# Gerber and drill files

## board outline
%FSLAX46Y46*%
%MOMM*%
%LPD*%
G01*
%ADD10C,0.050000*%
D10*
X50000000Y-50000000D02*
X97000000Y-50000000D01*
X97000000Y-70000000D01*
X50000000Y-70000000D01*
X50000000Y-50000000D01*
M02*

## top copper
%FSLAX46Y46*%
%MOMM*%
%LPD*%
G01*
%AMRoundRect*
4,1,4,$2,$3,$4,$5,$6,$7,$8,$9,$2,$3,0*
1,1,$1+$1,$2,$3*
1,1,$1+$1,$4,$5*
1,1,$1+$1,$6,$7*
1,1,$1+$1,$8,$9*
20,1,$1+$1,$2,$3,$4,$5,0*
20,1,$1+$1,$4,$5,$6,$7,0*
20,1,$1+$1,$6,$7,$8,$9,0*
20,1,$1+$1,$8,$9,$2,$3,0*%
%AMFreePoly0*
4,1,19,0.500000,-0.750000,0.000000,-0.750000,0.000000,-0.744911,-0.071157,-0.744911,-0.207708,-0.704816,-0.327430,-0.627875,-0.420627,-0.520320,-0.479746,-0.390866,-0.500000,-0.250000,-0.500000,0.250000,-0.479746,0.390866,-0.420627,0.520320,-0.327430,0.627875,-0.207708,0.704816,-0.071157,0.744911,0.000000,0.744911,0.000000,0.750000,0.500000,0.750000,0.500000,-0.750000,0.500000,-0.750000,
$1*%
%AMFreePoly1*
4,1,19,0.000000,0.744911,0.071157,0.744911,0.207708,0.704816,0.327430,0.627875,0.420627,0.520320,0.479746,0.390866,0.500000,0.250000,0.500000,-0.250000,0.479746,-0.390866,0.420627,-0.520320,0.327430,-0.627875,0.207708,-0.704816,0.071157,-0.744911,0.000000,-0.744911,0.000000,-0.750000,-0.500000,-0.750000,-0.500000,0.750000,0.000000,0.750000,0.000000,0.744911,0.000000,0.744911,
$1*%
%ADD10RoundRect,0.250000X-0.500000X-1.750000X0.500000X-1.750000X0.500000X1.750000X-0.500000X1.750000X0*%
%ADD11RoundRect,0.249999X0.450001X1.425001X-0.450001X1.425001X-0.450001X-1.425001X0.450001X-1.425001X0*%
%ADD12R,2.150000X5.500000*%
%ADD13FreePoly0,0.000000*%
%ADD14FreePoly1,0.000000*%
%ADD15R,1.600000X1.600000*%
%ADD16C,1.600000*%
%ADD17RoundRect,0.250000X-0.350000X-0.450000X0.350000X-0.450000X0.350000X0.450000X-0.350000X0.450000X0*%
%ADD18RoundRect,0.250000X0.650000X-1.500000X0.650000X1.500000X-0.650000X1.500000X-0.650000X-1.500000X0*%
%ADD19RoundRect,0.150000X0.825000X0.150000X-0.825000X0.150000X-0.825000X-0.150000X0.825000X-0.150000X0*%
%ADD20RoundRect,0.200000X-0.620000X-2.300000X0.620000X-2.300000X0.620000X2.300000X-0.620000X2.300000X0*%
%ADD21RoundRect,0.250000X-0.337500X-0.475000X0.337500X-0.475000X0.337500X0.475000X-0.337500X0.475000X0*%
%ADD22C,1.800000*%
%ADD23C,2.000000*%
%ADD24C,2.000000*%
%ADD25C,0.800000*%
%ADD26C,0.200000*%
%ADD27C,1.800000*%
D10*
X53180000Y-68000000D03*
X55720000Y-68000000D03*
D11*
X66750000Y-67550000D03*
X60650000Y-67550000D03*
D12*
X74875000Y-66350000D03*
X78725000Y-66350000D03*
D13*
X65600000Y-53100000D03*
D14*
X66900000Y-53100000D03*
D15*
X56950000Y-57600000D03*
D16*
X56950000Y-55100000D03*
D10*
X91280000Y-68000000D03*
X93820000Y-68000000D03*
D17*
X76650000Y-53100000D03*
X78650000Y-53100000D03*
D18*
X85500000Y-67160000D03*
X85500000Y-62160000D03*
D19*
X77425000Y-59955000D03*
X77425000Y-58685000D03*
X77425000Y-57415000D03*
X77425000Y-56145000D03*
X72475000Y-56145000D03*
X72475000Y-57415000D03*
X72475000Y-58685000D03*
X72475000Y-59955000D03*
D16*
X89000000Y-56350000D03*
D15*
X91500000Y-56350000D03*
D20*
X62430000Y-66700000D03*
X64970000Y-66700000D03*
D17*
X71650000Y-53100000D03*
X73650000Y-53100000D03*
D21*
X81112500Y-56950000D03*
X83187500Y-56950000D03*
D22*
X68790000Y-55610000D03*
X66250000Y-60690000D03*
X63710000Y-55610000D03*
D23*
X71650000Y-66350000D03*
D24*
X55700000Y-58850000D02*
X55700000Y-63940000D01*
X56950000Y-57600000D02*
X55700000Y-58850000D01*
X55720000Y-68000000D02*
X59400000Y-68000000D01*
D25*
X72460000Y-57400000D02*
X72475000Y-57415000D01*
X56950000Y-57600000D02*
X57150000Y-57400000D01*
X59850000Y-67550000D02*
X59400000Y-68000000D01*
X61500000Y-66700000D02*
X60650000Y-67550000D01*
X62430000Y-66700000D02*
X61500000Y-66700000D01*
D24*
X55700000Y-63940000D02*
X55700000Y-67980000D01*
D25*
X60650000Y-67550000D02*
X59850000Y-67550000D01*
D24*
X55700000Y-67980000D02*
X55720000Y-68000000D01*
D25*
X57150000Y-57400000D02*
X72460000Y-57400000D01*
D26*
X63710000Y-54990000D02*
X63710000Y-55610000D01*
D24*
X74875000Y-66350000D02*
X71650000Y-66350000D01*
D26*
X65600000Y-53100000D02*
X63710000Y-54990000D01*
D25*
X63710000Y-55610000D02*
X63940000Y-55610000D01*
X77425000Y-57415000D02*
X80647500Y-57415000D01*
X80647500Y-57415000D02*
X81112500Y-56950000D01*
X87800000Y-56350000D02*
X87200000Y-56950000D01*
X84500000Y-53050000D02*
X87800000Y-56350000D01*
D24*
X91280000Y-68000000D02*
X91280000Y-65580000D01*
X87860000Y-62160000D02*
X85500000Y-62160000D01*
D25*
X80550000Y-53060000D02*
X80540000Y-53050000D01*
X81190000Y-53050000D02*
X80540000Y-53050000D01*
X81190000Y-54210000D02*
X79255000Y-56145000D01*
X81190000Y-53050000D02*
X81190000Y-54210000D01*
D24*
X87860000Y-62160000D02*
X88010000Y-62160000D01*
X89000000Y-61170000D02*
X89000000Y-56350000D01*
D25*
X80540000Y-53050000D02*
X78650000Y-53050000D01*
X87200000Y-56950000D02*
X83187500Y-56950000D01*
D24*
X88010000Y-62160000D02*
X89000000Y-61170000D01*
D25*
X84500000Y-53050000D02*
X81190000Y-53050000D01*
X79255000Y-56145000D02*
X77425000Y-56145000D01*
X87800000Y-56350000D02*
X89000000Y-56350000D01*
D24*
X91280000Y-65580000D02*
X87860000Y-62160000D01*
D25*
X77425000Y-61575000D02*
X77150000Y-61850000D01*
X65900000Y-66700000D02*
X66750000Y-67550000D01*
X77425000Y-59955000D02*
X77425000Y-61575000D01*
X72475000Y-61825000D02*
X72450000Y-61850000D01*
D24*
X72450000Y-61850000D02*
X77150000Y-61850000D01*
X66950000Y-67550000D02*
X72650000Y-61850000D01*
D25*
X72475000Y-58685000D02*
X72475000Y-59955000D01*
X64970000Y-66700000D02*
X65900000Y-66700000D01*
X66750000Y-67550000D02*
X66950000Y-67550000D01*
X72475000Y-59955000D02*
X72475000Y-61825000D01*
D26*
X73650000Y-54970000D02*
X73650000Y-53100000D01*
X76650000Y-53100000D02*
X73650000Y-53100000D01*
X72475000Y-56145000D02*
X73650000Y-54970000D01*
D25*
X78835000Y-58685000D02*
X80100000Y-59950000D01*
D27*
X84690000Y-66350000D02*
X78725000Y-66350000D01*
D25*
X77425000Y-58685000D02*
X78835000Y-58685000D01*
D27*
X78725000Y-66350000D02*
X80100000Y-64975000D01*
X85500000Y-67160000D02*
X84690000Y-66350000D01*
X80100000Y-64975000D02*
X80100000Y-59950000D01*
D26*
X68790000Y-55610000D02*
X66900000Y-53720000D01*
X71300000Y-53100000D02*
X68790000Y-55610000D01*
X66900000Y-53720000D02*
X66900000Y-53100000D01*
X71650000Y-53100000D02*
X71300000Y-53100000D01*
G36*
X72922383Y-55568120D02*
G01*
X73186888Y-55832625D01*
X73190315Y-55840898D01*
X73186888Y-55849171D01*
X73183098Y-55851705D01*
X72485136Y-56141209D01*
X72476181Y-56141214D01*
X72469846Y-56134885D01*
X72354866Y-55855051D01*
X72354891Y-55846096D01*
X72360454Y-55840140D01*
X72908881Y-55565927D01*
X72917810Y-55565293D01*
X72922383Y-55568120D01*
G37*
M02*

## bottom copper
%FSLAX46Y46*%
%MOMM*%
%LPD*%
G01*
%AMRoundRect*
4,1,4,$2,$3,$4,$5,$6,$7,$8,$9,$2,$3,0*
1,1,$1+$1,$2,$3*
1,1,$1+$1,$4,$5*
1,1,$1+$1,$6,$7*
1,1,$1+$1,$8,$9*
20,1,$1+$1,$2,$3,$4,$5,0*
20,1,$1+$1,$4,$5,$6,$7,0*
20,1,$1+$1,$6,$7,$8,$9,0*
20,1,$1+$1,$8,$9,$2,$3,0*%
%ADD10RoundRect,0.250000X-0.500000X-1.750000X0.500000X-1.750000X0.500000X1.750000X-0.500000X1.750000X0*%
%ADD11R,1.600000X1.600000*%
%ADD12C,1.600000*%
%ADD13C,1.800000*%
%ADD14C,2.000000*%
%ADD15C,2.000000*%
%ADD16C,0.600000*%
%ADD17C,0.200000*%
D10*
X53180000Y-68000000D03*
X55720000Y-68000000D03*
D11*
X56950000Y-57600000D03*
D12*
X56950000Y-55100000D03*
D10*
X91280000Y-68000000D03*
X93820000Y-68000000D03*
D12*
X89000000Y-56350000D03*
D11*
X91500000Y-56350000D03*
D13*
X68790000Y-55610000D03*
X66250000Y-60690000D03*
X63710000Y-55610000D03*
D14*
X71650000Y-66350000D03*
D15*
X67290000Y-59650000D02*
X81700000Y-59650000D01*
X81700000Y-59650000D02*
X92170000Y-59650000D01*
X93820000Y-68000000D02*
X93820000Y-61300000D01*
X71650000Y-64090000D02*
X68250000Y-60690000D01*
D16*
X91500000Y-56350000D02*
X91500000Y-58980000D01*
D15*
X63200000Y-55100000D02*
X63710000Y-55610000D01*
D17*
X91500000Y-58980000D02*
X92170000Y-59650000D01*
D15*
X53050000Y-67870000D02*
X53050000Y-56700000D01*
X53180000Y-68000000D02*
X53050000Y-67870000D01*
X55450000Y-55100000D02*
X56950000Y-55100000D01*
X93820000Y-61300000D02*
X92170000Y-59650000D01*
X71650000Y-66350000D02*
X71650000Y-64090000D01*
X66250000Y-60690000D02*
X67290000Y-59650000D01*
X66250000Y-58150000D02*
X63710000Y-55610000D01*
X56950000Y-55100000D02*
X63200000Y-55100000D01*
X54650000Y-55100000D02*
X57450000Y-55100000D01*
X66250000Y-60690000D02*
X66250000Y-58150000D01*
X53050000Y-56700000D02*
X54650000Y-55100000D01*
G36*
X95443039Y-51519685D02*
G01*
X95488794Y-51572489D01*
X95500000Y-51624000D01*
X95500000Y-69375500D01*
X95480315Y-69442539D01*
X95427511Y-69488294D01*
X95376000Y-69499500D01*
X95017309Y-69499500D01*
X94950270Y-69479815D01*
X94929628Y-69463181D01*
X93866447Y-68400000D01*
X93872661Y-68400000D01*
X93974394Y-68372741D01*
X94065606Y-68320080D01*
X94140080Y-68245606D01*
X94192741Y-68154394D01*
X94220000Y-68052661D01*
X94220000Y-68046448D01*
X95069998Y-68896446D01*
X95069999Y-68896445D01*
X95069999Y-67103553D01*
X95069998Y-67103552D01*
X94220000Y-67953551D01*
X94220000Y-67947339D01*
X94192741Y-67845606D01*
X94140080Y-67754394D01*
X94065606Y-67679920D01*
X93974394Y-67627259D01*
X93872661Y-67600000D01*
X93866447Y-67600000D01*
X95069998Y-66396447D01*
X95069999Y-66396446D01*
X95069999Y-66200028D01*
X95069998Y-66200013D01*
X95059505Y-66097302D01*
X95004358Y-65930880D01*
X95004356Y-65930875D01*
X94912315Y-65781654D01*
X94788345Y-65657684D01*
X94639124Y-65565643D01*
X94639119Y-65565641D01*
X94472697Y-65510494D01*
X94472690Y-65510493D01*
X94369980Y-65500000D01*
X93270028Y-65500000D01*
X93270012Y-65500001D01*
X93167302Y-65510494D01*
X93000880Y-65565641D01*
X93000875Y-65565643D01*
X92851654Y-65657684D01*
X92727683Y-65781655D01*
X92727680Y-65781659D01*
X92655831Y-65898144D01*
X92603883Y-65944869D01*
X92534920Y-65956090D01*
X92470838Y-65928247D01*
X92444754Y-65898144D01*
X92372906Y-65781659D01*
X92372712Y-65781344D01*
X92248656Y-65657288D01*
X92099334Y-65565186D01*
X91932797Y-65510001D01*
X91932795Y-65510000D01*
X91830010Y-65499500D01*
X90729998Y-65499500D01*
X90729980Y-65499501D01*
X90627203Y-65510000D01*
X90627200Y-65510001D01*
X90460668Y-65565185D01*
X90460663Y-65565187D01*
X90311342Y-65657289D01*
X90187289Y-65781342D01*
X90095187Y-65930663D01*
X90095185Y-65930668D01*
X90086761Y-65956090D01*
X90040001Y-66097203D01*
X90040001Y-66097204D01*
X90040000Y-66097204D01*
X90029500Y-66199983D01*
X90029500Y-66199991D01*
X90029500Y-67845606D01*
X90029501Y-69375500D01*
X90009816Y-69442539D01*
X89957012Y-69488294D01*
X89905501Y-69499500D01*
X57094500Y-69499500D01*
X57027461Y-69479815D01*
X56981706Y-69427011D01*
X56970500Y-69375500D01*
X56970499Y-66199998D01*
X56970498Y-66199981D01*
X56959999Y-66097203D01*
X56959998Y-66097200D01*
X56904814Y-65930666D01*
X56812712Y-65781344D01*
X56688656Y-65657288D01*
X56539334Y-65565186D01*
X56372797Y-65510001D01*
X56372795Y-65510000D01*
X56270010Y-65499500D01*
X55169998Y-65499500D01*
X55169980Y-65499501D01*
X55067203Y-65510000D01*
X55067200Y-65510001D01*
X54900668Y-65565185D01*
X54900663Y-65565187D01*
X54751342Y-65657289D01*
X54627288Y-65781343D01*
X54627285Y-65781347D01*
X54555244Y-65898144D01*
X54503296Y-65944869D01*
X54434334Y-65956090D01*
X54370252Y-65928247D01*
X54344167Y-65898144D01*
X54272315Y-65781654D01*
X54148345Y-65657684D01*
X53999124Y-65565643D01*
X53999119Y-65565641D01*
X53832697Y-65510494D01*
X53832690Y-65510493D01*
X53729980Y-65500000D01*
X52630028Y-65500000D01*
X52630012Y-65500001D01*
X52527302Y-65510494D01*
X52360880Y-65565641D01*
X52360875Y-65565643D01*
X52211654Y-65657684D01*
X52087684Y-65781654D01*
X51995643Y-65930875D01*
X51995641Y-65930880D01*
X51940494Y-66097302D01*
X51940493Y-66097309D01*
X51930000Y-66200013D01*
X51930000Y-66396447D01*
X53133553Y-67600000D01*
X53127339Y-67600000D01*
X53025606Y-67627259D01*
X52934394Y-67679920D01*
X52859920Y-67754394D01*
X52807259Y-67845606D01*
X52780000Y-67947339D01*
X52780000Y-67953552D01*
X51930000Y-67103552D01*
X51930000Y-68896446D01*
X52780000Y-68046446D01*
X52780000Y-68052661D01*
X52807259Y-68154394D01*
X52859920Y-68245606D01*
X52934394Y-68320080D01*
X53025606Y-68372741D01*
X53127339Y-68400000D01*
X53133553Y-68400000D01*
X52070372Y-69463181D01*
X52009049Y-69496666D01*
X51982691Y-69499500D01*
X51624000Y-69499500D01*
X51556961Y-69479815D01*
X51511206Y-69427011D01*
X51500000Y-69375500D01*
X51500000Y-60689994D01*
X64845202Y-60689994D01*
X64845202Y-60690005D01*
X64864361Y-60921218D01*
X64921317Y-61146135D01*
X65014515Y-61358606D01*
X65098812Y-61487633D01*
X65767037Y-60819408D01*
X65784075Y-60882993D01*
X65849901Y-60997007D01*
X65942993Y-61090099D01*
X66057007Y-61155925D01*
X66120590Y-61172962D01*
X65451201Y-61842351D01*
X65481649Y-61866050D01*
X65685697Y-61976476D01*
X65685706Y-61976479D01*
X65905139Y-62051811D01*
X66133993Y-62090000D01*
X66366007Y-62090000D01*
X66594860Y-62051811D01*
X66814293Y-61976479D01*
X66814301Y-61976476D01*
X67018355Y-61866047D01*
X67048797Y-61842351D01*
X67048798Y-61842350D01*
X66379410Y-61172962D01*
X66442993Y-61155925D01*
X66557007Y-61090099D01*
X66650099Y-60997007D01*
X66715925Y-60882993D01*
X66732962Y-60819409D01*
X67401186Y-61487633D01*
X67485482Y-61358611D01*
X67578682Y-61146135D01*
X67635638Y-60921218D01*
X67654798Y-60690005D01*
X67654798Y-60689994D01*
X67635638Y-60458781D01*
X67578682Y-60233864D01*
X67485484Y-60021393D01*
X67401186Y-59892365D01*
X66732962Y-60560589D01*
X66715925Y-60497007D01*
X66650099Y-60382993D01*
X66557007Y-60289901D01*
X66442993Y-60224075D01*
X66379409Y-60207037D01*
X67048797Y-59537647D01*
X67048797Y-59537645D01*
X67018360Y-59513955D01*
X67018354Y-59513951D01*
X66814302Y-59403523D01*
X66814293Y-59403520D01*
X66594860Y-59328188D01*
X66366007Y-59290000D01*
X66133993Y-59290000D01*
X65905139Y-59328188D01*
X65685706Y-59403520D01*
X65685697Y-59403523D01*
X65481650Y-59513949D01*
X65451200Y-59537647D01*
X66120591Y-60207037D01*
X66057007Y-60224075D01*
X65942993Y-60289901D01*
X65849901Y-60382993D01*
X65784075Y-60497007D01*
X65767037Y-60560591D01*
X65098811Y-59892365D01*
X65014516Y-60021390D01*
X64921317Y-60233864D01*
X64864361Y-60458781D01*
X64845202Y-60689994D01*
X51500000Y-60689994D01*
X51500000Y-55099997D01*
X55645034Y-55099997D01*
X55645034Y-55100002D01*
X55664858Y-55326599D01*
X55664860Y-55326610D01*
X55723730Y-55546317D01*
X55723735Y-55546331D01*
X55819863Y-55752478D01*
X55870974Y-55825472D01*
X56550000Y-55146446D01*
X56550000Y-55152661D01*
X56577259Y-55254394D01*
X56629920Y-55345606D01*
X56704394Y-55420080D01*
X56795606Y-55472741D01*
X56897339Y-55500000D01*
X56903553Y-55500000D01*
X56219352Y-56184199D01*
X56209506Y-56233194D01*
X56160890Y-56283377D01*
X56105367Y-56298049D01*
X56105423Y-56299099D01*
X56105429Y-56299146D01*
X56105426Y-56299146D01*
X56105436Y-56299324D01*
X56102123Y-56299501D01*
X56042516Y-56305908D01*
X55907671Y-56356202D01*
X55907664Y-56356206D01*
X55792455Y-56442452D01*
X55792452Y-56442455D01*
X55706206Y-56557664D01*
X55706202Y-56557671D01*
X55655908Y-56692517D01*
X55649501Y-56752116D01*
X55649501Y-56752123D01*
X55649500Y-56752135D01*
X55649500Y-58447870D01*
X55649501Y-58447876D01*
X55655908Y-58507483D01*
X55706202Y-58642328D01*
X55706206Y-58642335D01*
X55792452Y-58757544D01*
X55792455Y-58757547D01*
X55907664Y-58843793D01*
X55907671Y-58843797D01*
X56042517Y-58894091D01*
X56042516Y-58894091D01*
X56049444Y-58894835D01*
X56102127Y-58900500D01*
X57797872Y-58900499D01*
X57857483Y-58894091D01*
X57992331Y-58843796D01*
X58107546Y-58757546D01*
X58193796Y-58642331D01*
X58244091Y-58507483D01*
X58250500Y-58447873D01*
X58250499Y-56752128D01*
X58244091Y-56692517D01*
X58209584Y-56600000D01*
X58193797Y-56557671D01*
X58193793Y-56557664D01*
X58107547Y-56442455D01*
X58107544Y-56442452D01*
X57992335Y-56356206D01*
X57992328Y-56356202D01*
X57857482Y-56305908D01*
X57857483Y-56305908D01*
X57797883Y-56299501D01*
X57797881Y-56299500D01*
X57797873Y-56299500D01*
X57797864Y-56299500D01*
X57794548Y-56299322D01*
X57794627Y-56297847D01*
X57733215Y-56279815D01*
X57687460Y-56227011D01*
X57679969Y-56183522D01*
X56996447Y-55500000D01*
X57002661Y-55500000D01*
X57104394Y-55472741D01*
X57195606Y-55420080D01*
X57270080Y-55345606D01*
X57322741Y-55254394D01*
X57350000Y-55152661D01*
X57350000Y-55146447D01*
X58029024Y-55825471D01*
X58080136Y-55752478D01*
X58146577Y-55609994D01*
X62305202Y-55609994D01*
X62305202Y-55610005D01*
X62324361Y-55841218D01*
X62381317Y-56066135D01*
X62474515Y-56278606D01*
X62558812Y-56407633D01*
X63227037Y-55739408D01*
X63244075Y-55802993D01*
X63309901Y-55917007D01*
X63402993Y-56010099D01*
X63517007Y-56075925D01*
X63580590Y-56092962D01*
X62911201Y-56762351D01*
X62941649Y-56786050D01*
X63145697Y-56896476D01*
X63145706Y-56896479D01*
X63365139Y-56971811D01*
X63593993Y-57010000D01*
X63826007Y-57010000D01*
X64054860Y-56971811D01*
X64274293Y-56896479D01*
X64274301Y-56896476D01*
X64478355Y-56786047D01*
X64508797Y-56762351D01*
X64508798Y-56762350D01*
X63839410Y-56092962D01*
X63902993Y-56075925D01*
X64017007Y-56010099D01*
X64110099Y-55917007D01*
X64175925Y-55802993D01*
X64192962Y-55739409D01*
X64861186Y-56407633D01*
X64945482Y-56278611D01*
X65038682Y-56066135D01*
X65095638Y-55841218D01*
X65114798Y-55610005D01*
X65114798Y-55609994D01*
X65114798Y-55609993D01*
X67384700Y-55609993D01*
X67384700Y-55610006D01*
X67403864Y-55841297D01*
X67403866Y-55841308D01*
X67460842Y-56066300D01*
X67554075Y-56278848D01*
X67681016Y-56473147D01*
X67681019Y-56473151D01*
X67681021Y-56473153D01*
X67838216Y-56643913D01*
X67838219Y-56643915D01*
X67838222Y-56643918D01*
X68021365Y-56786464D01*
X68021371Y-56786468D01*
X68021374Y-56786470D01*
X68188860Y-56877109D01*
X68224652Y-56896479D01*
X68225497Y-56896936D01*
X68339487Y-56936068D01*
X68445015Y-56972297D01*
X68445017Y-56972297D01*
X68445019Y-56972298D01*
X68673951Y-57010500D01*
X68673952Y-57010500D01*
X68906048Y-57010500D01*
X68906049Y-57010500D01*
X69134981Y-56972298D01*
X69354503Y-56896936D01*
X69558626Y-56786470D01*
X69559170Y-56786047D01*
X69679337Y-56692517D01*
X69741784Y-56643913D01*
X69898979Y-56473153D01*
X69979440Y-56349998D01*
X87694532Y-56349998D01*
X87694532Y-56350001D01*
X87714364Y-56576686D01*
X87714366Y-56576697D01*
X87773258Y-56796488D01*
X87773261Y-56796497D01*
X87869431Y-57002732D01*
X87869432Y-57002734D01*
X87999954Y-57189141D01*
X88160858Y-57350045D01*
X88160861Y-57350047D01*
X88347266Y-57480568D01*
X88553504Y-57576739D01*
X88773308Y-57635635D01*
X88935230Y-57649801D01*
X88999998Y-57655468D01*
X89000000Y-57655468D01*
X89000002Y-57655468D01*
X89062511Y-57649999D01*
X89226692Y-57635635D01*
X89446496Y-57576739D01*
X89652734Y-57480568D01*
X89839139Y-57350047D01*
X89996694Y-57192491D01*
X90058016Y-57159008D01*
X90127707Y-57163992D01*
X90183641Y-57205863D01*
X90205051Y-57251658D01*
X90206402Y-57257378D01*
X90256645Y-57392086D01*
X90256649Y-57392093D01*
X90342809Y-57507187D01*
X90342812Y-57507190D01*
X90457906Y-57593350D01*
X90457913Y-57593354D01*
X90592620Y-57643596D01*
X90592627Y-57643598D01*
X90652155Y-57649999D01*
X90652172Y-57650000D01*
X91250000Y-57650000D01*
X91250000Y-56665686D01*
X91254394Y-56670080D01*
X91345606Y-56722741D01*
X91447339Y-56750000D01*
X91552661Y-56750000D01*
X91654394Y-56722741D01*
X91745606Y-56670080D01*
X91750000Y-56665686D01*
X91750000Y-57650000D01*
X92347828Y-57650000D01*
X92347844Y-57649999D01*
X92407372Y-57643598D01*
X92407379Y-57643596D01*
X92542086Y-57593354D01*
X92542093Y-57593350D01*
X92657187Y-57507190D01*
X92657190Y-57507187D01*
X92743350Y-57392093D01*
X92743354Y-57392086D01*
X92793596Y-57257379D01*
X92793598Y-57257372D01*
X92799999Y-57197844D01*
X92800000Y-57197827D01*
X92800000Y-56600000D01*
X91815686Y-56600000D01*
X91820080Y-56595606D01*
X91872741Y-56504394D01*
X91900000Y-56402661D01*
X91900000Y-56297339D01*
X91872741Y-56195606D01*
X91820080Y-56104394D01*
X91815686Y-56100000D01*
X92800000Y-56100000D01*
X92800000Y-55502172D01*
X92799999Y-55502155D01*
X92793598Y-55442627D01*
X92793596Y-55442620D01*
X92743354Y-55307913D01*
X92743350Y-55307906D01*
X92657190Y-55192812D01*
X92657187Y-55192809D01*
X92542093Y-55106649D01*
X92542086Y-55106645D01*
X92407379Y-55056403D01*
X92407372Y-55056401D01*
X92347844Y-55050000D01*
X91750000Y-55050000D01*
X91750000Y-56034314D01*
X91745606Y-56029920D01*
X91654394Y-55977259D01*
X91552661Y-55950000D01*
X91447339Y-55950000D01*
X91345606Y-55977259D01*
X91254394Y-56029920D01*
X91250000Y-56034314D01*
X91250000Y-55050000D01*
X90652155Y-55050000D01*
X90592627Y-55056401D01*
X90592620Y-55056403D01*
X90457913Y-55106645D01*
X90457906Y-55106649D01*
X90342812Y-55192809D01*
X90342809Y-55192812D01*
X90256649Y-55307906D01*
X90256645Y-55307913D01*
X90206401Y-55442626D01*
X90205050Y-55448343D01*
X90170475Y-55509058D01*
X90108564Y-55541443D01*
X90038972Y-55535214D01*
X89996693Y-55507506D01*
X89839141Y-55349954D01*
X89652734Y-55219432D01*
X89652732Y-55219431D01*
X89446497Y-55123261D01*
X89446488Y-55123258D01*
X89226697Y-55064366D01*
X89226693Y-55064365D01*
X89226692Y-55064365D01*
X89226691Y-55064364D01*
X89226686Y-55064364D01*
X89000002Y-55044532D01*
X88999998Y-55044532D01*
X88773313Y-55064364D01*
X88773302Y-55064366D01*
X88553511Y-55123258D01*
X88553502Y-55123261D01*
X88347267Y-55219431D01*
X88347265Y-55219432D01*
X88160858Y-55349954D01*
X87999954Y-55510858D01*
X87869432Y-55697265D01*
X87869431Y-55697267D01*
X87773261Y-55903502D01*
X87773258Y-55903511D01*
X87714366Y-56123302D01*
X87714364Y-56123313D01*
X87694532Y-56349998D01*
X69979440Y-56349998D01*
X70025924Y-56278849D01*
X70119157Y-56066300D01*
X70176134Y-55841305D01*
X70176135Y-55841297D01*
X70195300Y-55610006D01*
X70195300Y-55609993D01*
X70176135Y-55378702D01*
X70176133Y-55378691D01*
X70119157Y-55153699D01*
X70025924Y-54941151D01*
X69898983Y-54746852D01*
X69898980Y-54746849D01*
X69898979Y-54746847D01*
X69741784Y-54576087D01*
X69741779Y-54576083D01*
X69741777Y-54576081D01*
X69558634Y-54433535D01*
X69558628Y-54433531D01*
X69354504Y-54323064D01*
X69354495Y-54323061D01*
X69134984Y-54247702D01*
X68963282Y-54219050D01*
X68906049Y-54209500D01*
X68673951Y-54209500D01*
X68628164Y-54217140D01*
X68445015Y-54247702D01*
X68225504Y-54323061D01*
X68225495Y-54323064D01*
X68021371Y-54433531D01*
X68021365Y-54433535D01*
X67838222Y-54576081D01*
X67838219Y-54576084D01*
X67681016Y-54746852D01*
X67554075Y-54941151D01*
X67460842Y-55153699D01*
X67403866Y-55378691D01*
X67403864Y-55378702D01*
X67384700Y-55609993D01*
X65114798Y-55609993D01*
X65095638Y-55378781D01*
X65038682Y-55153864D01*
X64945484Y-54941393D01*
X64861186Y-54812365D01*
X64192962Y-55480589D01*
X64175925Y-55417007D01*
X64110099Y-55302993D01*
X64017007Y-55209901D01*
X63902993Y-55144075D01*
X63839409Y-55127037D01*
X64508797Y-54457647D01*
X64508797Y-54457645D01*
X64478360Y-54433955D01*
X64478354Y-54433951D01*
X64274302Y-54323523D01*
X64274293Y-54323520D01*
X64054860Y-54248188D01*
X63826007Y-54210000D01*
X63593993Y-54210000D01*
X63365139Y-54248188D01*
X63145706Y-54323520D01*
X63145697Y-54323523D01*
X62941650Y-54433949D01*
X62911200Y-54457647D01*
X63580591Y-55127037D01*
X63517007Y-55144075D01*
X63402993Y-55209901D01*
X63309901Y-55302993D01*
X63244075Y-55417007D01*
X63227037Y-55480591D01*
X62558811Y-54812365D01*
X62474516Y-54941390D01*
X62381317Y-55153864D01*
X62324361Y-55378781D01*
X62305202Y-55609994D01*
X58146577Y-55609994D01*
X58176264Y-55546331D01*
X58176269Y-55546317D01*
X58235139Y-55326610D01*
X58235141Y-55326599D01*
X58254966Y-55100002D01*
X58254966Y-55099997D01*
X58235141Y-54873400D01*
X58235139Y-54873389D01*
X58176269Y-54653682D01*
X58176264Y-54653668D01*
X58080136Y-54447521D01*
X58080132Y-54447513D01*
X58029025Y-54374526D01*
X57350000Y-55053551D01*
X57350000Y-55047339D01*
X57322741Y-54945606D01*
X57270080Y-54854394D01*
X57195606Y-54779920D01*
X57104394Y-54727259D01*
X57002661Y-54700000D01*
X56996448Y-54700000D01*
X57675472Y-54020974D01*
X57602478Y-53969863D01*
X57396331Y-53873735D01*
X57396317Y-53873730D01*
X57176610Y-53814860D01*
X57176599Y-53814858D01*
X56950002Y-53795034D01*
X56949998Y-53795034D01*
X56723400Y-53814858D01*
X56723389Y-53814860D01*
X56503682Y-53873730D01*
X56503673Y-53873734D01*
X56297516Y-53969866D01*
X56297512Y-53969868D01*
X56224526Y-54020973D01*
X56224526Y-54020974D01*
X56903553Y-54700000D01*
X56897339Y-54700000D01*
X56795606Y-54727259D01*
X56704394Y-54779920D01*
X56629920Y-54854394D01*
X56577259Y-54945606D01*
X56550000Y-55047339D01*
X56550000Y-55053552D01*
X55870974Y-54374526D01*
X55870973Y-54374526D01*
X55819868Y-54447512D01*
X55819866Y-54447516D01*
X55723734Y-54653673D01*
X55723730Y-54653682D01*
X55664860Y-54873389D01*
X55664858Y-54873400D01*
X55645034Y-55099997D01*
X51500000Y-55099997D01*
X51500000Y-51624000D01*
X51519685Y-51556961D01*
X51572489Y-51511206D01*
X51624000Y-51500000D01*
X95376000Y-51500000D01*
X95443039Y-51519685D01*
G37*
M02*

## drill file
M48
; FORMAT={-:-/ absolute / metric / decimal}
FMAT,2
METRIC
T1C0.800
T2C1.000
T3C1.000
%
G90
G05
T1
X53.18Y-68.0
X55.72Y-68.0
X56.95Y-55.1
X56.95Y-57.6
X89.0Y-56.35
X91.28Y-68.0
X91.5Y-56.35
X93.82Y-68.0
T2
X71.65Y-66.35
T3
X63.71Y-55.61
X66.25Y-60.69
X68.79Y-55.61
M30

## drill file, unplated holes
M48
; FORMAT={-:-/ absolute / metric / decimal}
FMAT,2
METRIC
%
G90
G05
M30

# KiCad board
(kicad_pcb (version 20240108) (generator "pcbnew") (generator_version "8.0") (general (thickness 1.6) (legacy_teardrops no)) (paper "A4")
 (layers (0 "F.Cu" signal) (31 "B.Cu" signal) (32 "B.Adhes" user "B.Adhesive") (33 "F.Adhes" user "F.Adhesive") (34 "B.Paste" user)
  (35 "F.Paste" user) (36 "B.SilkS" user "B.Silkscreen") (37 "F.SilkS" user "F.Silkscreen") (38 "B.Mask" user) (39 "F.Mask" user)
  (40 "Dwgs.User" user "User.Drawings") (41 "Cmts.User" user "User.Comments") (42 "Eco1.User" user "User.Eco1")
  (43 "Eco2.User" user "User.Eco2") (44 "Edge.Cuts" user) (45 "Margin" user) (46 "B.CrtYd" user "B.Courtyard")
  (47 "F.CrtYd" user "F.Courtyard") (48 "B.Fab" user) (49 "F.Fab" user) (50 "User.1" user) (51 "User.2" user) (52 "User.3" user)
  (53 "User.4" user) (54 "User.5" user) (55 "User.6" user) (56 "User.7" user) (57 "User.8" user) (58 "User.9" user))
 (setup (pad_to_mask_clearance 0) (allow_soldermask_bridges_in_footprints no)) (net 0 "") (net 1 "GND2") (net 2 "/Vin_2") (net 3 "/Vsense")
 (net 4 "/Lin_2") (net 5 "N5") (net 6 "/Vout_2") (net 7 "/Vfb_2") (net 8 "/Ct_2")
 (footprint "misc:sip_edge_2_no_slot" (layer "F.Cu") (at 54.45 70)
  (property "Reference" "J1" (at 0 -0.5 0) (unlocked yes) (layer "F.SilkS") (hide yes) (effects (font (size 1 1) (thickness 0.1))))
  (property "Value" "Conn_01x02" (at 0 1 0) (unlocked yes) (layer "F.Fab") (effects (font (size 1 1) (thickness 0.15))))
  (pad "1" thru_hole roundrect (at -1.27 -2) (size 1.5 4) (drill 0.8) (layers "*.Cu" "*.Mask") (remove_unused_layers no)
   (roundrect_rratio 0.1666666667) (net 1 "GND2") (thermal_bridge_angle 45))
  (pad "2" thru_hole roundrect (at 1.27 -2) (size 1.5 4) (drill 0.8) (layers "*.Cu" "*.Mask") (remove_unused_layers no)
   (roundrect_rratio 0.1666666667) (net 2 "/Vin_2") (thermal_bridge_angle 45)))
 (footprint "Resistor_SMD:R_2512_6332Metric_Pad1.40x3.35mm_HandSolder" (layer "F.Cu") (at 63.7 67.55 180)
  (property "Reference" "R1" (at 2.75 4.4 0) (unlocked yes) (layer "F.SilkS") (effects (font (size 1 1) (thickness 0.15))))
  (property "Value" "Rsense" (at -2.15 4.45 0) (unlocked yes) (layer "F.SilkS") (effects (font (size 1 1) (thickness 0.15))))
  (pad "1" smd roundrect (at -3.05 0 180) (size 1.4 3.35) (layers "F.Cu" "F.Paste" "F.Mask") (roundrect_rratio 0.178571) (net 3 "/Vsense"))
  (pad "2" smd roundrect (at 3.05 0 180) (size 1.4 3.35) (layers "F.Cu" "F.Paste" "F.Mask") (roundrect_rratio 0.178571) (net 2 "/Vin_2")))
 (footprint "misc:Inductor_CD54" (layer "F.Cu") (at 76.8 66.35 90)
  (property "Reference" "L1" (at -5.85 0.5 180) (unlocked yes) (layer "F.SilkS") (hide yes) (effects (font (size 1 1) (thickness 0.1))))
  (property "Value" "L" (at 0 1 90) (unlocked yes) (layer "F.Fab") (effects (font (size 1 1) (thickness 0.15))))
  (pad "1" smd rect (at 0 -1.925 90) (size 5.5 2.15) (layers "F.Cu" "F.Paste" "F.Mask") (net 1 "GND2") (thermal_bridge_angle 45))
  (pad "2" smd rect (at 0 1.925 90) (size 5.5 2.15) (layers "F.Cu" "F.Paste" "F.Mask") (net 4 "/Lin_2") (thermal_bridge_angle 45)))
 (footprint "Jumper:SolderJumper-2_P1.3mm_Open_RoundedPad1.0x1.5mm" (layer "F.Cu") (at 66.25 53.1)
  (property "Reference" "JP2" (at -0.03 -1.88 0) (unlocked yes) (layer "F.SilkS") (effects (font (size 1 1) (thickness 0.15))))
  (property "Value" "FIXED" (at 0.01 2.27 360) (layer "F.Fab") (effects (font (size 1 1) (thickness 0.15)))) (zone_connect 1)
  (pad "1" smd custom (at -0.65 0) (size 1 0.5) (layers "F.Cu" "F.Mask") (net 1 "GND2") (zone_connect 2) (thermal_bridge_angle 45)
   (options (clearance outline) (anchor rect)) (primitives))
  (pad "2" smd custom (at 0.65 0) (size 1 0.5) (layers "F.Cu" "F.Mask") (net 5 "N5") (zone_connect 2) (thermal_bridge_angle 45)
   (options (clearance outline) (anchor rect)) (primitives)))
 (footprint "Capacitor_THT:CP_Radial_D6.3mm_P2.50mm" (layer "F.Cu") (at 56.95 57.6 90)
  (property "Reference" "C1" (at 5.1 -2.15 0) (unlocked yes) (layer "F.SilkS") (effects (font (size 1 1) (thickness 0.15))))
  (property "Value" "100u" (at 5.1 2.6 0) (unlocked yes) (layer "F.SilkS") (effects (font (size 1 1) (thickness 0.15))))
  (pad "1" thru_hole rect (at 0 0 90) (size 1.6 1.6) (drill 0.8) (layers "*.Cu" "*.Mask") (remove_unused_layers no) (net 2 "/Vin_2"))
  (pad "2" thru_hole circle (at 2.5 0 90) (size 1.6 1.6) (drill 0.8) (layers "*.Cu" "*.Mask") (remove_unused_layers no) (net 1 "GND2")))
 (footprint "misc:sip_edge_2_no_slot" (layer "F.Cu") (at 92.55 70)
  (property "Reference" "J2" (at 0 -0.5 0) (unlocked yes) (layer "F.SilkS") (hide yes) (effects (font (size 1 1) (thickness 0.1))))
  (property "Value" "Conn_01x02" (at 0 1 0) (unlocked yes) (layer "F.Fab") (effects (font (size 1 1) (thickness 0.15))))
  (pad "1" thru_hole roundrect (at -1.27 -2) (size 1.5 4) (drill 0.8) (layers "*.Cu" "*.Mask") (remove_unused_layers no)
   (roundrect_rratio 0.1666666667) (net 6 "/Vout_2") (thermal_bridge_angle 45))
  (pad "2" thru_hole roundrect (at 1.27 -2) (size 1.5 4) (drill 0.8) (layers "*.Cu" "*.Mask") (remove_unused_layers no)
   (roundrect_rratio 0.1666666667) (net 1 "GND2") (thermal_bridge_angle 45)))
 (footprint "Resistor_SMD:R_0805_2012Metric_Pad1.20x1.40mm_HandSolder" (layer "F.Cu") (at 77.65 53.1)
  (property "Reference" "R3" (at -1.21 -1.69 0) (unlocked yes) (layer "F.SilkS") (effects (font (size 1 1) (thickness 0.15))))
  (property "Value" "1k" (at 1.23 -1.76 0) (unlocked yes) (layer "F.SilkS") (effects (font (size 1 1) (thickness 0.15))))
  (pad "1" smd roundrect (at -1 0) (size 1.2 1.4) (layers "F.Cu" "F.Paste" "F.Mask") (roundrect_rratio 0.208333) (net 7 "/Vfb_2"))
  (pad "2" smd roundrect (at 1 0) (size 1.2 1.4) (layers "F.Cu" "F.Paste" "F.Mask") (roundrect_rratio 0.208333) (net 6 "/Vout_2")))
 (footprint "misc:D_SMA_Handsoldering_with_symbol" (layer "F.Cu") (at 85.5 64.66 90)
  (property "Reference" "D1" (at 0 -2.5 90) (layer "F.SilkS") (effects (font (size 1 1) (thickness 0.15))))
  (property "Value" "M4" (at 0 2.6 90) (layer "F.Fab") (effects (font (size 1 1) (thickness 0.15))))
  (pad "1" smd roundrect (at -2.5 0 90) (size 3.5 1.8) (layers "F.Cu" "F.Paste" "F.Mask") (roundrect_rratio 0.1388888889) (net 4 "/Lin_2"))
  (pad "2" smd roundrect (at 2.5 0 90) (size 3.5 1.8) (layers "F.Cu" "F.Paste" "F.Mask") (roundrect_rratio 0.1388888889) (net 6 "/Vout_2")))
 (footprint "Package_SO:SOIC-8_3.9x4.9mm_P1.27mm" (layer "F.Cu") (at 74.95 58.05 180)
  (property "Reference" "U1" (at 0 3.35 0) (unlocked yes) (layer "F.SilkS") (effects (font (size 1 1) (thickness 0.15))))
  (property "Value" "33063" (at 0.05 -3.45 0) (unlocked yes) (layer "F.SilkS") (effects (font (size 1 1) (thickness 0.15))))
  (pad "1" smd roundrect (at -2.475 -1.905 180) (size 1.95 0.6) (layers "F.Cu" "F.Paste" "F.Mask") (roundrect_rratio 0.25) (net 3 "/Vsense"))
  (pad "2" smd roundrect (at -2.475 -0.635 180) (size 1.95 0.6) (layers "F.Cu" "F.Paste" "F.Mask") (roundrect_rratio 0.25) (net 4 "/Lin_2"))
  (pad "3" smd roundrect (at -2.475 0.635 180) (size 1.95 0.6) (layers "F.Cu" "F.Paste" "F.Mask") (roundrect_rratio 0.25) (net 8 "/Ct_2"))
  (pad "4" smd roundrect (at -2.475 1.905 180) (size 1.95 0.6) (layers "F.Cu" "F.Paste" "F.Mask") (roundrect_rratio 0.25) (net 6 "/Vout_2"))
  (pad "5" smd roundrect (at 2.475 1.905 180) (size 1.95 0.6) (layers "F.Cu" "F.Paste" "F.Mask") (roundrect_rratio 0.25) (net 7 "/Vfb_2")
   (teardrops (best_length_ratio 0.5) (max_length 1) (best_width_ratio 1) (max_width 2) (curve_points 0) (filter_ratio 0.9) (enabled yes)
    (allow_two_segments yes) (prefer_zone_connections yes)))
  (pad "6" smd roundrect (at 2.475 0.635 180) (size 1.95 0.6) (layers "F.Cu" "F.Paste" "F.Mask") (roundrect_rratio 0.25) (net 2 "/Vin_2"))
  (pad "7" smd roundrect (at 2.475 -0.635 180) (size 1.95 0.6) (layers "F.Cu" "F.Paste" "F.Mask") (roundrect_rratio 0.25) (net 3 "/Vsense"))
  (pad "8" smd roundrect (at 2.475 -1.905 180) (size 1.95 0.6) (layers "F.Cu" "F.Paste" "F.Mask") (roundrect_rratio 0.25) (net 3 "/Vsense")))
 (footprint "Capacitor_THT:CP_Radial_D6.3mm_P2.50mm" (layer "F.Cu") (at 91.5 56.35 180)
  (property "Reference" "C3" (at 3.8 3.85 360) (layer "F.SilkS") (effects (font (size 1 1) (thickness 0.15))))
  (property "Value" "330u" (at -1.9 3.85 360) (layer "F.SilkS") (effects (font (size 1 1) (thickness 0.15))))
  (pad "1" thru_hole rect (at 0 0 180) (size 1.6 1.6) (drill 0.8) (layers "*.Cu" "*.Mask") (remove_unused_layers no) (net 1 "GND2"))
  (pad "2" thru_hole circle (at 2.5 0 180) (size 1.6 1.6) (drill 0.8) (layers "*.Cu" "*.Mask") (remove_unused_layers no) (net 6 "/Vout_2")))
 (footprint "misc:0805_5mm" (layer "F.Cu") (at 63.7 66.7)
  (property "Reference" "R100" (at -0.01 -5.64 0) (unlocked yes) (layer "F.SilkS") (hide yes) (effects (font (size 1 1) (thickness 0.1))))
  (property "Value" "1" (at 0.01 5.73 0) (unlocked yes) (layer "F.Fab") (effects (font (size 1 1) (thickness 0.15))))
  (pad "1" smd roundrect (at -1.27 0) (size 1.64 5) (layers "F.Cu" "F.Paste" "F.Mask") (roundrect_rratio 0.1219512195) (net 2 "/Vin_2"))
  (pad "2" smd roundrect (at 1.27 0) (size 1.64 5) (layers "F.Cu" "F.Paste" "F.Mask") (roundrect_rratio 0.1219512195) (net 3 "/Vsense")))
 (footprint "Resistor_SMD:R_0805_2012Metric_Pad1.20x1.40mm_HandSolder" (layer "F.Cu") (at 72.65 53.1)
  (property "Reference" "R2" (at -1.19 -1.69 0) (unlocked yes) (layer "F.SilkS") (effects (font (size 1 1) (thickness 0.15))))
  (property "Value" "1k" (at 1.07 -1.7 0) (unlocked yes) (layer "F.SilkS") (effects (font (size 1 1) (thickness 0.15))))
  (pad "1" smd roundrect (at -1 0) (size 1.2 1.4) (layers "F.Cu" "F.Paste" "F.Mask") (roundrect_rratio 0.208333) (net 5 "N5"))
  (pad "2" smd roundrect (at 1 0) (size 1.2 1.4) (layers "F.Cu" "F.Paste" "F.Mask") (roundrect_rratio 0.208333) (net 7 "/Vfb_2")))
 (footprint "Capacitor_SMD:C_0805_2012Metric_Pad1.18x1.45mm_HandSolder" (layer "F.Cu") (at 82.15 56.95)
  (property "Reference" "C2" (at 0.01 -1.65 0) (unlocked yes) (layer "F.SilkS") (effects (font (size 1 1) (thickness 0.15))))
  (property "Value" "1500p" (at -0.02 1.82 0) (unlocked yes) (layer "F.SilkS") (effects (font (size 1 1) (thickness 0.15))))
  (pad "1" smd roundrect (at -1.0375 0) (size 1.175 1.45) (layers "F.Cu" "F.Paste" "F.Mask") (roundrect_rratio 0.212766) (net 8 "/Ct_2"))
  (pad "2" smd roundrect (at 1.0375 0) (size 1.175 1.45) (layers "F.Cu" "F.Paste" "F.Mask") (roundrect_rratio 0.212766) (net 6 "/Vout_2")))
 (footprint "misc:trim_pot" (layer "F.Cu") (at 66.25 58.15 180)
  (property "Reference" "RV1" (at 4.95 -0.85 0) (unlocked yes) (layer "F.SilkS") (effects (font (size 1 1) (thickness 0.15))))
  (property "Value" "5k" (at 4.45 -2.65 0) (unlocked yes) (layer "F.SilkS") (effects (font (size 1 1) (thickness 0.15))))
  (pad "1" thru_hole circle (at -2.54 2.54 180) (size 1.8 1.8) (drill 1) (layers "*.Cu" "*.Mask") (remove_unused_layers no) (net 5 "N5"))
  (pad "2" thru_hole circle (at 0 -2.54 180) (size 1.8 1.8) (drill 1) (layers "*.Cu" "*.Mask") (remove_unused_layers no) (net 1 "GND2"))
  (pad "3" thru_hole circle (at 2.54 2.54 180) (size 1.8 1.8) (drill 1) (layers "*.Cu" "*.Mask") (remove_unused_layers no) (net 1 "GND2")))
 (gr_rect (start 50 50) (end 97 70) (stroke (width 0.05) (type default)) (fill none) (layer "Edge.Cuts"))
 (segment (start 55.7 58.85) (end 55.7 63.94) (width 2) (layer "F.Cu") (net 2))
 (segment (start 56.95 57.6) (end 55.7 58.85) (width 2) (layer "F.Cu") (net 2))
 (segment (start 55.72 68) (end 59.4 68) (width 2) (layer "F.Cu") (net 2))
 (segment (start 72.46 57.4) (end 72.475 57.415) (width 0.8) (layer "F.Cu") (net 2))
 (segment (start 56.95 57.6) (end 57.15 57.4) (width 0.8) (layer "F.Cu") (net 2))
 (segment (start 59.85 67.55) (end 59.4 68) (width 0.8) (layer "F.Cu") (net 2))
 (segment (start 61.5 66.7) (end 60.65 67.55) (width 0.8) (layer "F.Cu") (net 2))
 (segment (start 62.43 66.7) (end 61.5 66.7) (width 0.8) (layer "F.Cu") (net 2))
 (segment (start 55.7 63.94) (end 55.7 67.98) (width 2) (layer "F.Cu") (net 2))
 (segment (start 60.65 67.55) (end 59.85 67.55) (width 0.8) (layer "F.Cu") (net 2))
 (segment (start 55.7 67.98) (end 55.72 68) (width 2) (layer "F.Cu") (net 2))
 (segment (start 57.15 57.4) (end 72.46 57.4) (width 0.8) (layer "F.Cu") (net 2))
 (segment (start 63.71 54.99) (end 63.71 55.61) (width 0.2) (layer "F.Cu") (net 1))
 (segment (start 74.875 66.35) (end 71.65 66.35) (width 2) (layer "F.Cu") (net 1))
 (segment (start 65.6 53.1) (end 63.71 54.99) (width 0.2) (layer "F.Cu") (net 1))
 (segment (start 63.71 55.61) (end 63.94 55.61) (width 0.8) (layer "F.Cu") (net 1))
 (via (at 71.65 66.35) (size 2) (drill 1) (layers "F.Cu" "B.Cu") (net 1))
 (segment (start 67.29 59.65) (end 81.7 59.65) (width 2) (layer "B.Cu") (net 1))
 (segment (start 81.7 59.65) (end 92.17 59.65) (width 2) (layer "B.Cu") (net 1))
 (segment (start 93.82 68) (end 93.82 61.3) (width 2) (layer "B.Cu") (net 1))
 (segment (start 71.65 64.09) (end 68.25 60.69) (width 2) (layer "B.Cu") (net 1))
 (segment (start 91.5 56.35) (end 91.5 58.98) (width 0.6) (layer "B.Cu") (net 1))
 (segment (start 63.2 55.1) (end 63.71 55.61) (width 2) (layer "B.Cu") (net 1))
 (segment (start 91.5 58.98) (end 92.17 59.65) (width 0.2) (layer "B.Cu") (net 1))
 (segment (start 53.05 67.87) (end 53.05 56.7) (width 2) (layer "B.Cu") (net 1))
 (segment (start 53.18 68) (end 53.05 67.87) (width 2) (layer "B.Cu") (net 1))
 (segment (start 55.45 55.1) (end 56.95 55.1) (width 2) (layer "B.Cu") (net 1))
 (segment (start 93.82 61.3) (end 92.17 59.65) (width 2) (layer "B.Cu") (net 1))
 (segment (start 71.65 66.35) (end 71.65 64.09) (width 2) (layer "B.Cu") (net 1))
 (segment (start 66.25 60.69) (end 67.29 59.65) (width 2) (layer "B.Cu") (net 1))
 (segment (start 66.25 58.15) (end 63.71 55.61) (width 2) (layer "B.Cu") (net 1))
 (segment (start 56.95 55.1) (end 63.2 55.1) (width 2) (layer "B.Cu") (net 1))
 (segment (start 54.65 55.1) (end 57.45 55.1) (width 2) (layer "B.Cu") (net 1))
 (segment (start 66.25 60.69) (end 66.25 58.15) (width 2) (layer "B.Cu") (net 1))
 (segment (start 53.05 56.7) (end 54.65 55.1) (width 2) (layer "B.Cu") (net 1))
 (segment (start 77.425 57.415) (end 80.6475 57.415) (width 0.8) (layer "F.Cu") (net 8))
 (segment (start 80.6475 57.415) (end 81.1125 56.95) (width 0.8) (layer "F.Cu") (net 8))
 (segment (start 87.8 56.35) (end 87.2 56.95) (width 0.8) (layer "F.Cu") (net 6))
 (segment (start 84.5 53.05) (end 87.8 56.35) (width 0.8) (layer "F.Cu") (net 6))
 (segment (start 91.28 68) (end 91.28 65.58) (width 2) (layer "F.Cu") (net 6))
 (segment (start 87.86 62.16) (end 85.5 62.16) (width 2) (layer "F.Cu") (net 6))
 (segment (start 80.55 53.06) (end 80.54 53.05) (width 0.8) (layer "F.Cu") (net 6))
 (segment (start 81.19 53.05) (end 80.54 53.05) (width 0.8) (layer "F.Cu") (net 6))
 (segment (start 81.19 54.21) (end 79.255 56.145) (width 0.8) (layer "F.Cu") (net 6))
 (segment (start 81.19 53.05) (end 81.19 54.21) (width 0.8) (layer "F.Cu") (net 6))
 (segment (start 87.86 62.16) (end 88.01 62.16) (width 2) (layer "F.Cu") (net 6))
 (segment (start 89 61.17) (end 89 56.35) (width 2) (layer "F.Cu") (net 6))
 (segment (start 80.54 53.05) (end 78.65 53.05) (width 0.8) (layer "F.Cu") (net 6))
 (segment (start 87.2 56.95) (end 83.1875 56.95) (width 0.8) (layer "F.Cu") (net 6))
 (segment (start 88.01 62.16) (end 89 61.17) (width 2) (layer "F.Cu") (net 6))
 (segment (start 84.5 53.05) (end 81.19 53.05) (width 0.8) (layer "F.Cu") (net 6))
 (segment (start 79.255 56.145) (end 77.425 56.145) (width 0.8) (layer "F.Cu") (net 6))
 (segment (start 87.8 56.35) (end 89 56.35) (width 0.8) (layer "F.Cu") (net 6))
 (segment (start 91.28 65.58) (end 87.86 62.16) (width 2) (layer "F.Cu") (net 6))
 (segment (start 77.425 61.575) (end 77.15 61.85) (width 0.8) (layer "F.Cu") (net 3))
 (segment (start 65.9 66.7) (end 66.75 67.55) (width 0.8) (layer "F.Cu") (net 3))
 (segment (start 77.425 59.955) (end 77.425 61.575) (width 0.8) (layer "F.Cu") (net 3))
 (segment (start 72.475 61.825) (end 72.45 61.85) (width 0.8) (layer "F.Cu") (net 3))
 (segment (start 72.45 61.85) (end 77.15 61.85) (width 2) (layer "F.Cu") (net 3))
 (segment (start 66.95 67.55) (end 72.65 61.85) (width 2) (layer "F.Cu") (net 3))
 (segment (start 72.475 58.685) (end 72.475 59.955) (width 0.8) (layer "F.Cu") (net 3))
 (segment (start 64.97 66.7) (end 65.9 66.7) (width 0.8) (layer "F.Cu") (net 3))
 (segment (start 66.75 67.55) (end 66.95 67.55) (width 0.8) (layer "F.Cu") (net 3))
 (segment (start 72.475 59.955) (end 72.475 61.825) (width 0.8) (layer "F.Cu") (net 3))
 (segment (start 73.65 54.97) (end 73.65 53.1) (width 0.2) (layer "F.Cu") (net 7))
 (segment (start 76.65 53.1) (end 73.65 53.1) (width 0.2) (layer "F.Cu") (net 7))
 (segment (start 72.475 56.145) (end 73.65 54.97) (width 0.2) (layer "F.Cu") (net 7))
 (segment (start 78.835 58.685) (end 80.1 59.95) (width 0.8) (layer "F.Cu") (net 4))
 (segment (start 84.69 66.35) (end 78.725 66.35) (width 1.8) (layer "F.Cu") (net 4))
 (segment (start 77.425 58.685) (end 78.835 58.685) (width 0.8) (layer "F.Cu") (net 4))
 (segment (start 78.725 66.35) (end 80.1 64.975) (width 1.8) (layer "F.Cu") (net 4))
 (segment (start 85.5 67.16) (end 84.69 66.35) (width 1.8) (layer "F.Cu") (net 4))
 (segment (start 80.1 64.975) (end 80.1 59.95) (width 1.8) (layer "F.Cu") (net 4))
 (segment (start 68.79 55.61) (end 66.9 53.72) (width 0.2) (layer "F.Cu") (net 5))
 (segment (start 71.3 53.1) (end 68.79 55.61) (width 0.2) (layer "F.Cu") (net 5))
 (segment (start 66.9 53.72) (end 66.9 53.1) (width 0.2) (layer "F.Cu") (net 5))
 (segment (start 71.65 53.1) (end 71.3 53.1) (width 0.2) (layer "F.Cu") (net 5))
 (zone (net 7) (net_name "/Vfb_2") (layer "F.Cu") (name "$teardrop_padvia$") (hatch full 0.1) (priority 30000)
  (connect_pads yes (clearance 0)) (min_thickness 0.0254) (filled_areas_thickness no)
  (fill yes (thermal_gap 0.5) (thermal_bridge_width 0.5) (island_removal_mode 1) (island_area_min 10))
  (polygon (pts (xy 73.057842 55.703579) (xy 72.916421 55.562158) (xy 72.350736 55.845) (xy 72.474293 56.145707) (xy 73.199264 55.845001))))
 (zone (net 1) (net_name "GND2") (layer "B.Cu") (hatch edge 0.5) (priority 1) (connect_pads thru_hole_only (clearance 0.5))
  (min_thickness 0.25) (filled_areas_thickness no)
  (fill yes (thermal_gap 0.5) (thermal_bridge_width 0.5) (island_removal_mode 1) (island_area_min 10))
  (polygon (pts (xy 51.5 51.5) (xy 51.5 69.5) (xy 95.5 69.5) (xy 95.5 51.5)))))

